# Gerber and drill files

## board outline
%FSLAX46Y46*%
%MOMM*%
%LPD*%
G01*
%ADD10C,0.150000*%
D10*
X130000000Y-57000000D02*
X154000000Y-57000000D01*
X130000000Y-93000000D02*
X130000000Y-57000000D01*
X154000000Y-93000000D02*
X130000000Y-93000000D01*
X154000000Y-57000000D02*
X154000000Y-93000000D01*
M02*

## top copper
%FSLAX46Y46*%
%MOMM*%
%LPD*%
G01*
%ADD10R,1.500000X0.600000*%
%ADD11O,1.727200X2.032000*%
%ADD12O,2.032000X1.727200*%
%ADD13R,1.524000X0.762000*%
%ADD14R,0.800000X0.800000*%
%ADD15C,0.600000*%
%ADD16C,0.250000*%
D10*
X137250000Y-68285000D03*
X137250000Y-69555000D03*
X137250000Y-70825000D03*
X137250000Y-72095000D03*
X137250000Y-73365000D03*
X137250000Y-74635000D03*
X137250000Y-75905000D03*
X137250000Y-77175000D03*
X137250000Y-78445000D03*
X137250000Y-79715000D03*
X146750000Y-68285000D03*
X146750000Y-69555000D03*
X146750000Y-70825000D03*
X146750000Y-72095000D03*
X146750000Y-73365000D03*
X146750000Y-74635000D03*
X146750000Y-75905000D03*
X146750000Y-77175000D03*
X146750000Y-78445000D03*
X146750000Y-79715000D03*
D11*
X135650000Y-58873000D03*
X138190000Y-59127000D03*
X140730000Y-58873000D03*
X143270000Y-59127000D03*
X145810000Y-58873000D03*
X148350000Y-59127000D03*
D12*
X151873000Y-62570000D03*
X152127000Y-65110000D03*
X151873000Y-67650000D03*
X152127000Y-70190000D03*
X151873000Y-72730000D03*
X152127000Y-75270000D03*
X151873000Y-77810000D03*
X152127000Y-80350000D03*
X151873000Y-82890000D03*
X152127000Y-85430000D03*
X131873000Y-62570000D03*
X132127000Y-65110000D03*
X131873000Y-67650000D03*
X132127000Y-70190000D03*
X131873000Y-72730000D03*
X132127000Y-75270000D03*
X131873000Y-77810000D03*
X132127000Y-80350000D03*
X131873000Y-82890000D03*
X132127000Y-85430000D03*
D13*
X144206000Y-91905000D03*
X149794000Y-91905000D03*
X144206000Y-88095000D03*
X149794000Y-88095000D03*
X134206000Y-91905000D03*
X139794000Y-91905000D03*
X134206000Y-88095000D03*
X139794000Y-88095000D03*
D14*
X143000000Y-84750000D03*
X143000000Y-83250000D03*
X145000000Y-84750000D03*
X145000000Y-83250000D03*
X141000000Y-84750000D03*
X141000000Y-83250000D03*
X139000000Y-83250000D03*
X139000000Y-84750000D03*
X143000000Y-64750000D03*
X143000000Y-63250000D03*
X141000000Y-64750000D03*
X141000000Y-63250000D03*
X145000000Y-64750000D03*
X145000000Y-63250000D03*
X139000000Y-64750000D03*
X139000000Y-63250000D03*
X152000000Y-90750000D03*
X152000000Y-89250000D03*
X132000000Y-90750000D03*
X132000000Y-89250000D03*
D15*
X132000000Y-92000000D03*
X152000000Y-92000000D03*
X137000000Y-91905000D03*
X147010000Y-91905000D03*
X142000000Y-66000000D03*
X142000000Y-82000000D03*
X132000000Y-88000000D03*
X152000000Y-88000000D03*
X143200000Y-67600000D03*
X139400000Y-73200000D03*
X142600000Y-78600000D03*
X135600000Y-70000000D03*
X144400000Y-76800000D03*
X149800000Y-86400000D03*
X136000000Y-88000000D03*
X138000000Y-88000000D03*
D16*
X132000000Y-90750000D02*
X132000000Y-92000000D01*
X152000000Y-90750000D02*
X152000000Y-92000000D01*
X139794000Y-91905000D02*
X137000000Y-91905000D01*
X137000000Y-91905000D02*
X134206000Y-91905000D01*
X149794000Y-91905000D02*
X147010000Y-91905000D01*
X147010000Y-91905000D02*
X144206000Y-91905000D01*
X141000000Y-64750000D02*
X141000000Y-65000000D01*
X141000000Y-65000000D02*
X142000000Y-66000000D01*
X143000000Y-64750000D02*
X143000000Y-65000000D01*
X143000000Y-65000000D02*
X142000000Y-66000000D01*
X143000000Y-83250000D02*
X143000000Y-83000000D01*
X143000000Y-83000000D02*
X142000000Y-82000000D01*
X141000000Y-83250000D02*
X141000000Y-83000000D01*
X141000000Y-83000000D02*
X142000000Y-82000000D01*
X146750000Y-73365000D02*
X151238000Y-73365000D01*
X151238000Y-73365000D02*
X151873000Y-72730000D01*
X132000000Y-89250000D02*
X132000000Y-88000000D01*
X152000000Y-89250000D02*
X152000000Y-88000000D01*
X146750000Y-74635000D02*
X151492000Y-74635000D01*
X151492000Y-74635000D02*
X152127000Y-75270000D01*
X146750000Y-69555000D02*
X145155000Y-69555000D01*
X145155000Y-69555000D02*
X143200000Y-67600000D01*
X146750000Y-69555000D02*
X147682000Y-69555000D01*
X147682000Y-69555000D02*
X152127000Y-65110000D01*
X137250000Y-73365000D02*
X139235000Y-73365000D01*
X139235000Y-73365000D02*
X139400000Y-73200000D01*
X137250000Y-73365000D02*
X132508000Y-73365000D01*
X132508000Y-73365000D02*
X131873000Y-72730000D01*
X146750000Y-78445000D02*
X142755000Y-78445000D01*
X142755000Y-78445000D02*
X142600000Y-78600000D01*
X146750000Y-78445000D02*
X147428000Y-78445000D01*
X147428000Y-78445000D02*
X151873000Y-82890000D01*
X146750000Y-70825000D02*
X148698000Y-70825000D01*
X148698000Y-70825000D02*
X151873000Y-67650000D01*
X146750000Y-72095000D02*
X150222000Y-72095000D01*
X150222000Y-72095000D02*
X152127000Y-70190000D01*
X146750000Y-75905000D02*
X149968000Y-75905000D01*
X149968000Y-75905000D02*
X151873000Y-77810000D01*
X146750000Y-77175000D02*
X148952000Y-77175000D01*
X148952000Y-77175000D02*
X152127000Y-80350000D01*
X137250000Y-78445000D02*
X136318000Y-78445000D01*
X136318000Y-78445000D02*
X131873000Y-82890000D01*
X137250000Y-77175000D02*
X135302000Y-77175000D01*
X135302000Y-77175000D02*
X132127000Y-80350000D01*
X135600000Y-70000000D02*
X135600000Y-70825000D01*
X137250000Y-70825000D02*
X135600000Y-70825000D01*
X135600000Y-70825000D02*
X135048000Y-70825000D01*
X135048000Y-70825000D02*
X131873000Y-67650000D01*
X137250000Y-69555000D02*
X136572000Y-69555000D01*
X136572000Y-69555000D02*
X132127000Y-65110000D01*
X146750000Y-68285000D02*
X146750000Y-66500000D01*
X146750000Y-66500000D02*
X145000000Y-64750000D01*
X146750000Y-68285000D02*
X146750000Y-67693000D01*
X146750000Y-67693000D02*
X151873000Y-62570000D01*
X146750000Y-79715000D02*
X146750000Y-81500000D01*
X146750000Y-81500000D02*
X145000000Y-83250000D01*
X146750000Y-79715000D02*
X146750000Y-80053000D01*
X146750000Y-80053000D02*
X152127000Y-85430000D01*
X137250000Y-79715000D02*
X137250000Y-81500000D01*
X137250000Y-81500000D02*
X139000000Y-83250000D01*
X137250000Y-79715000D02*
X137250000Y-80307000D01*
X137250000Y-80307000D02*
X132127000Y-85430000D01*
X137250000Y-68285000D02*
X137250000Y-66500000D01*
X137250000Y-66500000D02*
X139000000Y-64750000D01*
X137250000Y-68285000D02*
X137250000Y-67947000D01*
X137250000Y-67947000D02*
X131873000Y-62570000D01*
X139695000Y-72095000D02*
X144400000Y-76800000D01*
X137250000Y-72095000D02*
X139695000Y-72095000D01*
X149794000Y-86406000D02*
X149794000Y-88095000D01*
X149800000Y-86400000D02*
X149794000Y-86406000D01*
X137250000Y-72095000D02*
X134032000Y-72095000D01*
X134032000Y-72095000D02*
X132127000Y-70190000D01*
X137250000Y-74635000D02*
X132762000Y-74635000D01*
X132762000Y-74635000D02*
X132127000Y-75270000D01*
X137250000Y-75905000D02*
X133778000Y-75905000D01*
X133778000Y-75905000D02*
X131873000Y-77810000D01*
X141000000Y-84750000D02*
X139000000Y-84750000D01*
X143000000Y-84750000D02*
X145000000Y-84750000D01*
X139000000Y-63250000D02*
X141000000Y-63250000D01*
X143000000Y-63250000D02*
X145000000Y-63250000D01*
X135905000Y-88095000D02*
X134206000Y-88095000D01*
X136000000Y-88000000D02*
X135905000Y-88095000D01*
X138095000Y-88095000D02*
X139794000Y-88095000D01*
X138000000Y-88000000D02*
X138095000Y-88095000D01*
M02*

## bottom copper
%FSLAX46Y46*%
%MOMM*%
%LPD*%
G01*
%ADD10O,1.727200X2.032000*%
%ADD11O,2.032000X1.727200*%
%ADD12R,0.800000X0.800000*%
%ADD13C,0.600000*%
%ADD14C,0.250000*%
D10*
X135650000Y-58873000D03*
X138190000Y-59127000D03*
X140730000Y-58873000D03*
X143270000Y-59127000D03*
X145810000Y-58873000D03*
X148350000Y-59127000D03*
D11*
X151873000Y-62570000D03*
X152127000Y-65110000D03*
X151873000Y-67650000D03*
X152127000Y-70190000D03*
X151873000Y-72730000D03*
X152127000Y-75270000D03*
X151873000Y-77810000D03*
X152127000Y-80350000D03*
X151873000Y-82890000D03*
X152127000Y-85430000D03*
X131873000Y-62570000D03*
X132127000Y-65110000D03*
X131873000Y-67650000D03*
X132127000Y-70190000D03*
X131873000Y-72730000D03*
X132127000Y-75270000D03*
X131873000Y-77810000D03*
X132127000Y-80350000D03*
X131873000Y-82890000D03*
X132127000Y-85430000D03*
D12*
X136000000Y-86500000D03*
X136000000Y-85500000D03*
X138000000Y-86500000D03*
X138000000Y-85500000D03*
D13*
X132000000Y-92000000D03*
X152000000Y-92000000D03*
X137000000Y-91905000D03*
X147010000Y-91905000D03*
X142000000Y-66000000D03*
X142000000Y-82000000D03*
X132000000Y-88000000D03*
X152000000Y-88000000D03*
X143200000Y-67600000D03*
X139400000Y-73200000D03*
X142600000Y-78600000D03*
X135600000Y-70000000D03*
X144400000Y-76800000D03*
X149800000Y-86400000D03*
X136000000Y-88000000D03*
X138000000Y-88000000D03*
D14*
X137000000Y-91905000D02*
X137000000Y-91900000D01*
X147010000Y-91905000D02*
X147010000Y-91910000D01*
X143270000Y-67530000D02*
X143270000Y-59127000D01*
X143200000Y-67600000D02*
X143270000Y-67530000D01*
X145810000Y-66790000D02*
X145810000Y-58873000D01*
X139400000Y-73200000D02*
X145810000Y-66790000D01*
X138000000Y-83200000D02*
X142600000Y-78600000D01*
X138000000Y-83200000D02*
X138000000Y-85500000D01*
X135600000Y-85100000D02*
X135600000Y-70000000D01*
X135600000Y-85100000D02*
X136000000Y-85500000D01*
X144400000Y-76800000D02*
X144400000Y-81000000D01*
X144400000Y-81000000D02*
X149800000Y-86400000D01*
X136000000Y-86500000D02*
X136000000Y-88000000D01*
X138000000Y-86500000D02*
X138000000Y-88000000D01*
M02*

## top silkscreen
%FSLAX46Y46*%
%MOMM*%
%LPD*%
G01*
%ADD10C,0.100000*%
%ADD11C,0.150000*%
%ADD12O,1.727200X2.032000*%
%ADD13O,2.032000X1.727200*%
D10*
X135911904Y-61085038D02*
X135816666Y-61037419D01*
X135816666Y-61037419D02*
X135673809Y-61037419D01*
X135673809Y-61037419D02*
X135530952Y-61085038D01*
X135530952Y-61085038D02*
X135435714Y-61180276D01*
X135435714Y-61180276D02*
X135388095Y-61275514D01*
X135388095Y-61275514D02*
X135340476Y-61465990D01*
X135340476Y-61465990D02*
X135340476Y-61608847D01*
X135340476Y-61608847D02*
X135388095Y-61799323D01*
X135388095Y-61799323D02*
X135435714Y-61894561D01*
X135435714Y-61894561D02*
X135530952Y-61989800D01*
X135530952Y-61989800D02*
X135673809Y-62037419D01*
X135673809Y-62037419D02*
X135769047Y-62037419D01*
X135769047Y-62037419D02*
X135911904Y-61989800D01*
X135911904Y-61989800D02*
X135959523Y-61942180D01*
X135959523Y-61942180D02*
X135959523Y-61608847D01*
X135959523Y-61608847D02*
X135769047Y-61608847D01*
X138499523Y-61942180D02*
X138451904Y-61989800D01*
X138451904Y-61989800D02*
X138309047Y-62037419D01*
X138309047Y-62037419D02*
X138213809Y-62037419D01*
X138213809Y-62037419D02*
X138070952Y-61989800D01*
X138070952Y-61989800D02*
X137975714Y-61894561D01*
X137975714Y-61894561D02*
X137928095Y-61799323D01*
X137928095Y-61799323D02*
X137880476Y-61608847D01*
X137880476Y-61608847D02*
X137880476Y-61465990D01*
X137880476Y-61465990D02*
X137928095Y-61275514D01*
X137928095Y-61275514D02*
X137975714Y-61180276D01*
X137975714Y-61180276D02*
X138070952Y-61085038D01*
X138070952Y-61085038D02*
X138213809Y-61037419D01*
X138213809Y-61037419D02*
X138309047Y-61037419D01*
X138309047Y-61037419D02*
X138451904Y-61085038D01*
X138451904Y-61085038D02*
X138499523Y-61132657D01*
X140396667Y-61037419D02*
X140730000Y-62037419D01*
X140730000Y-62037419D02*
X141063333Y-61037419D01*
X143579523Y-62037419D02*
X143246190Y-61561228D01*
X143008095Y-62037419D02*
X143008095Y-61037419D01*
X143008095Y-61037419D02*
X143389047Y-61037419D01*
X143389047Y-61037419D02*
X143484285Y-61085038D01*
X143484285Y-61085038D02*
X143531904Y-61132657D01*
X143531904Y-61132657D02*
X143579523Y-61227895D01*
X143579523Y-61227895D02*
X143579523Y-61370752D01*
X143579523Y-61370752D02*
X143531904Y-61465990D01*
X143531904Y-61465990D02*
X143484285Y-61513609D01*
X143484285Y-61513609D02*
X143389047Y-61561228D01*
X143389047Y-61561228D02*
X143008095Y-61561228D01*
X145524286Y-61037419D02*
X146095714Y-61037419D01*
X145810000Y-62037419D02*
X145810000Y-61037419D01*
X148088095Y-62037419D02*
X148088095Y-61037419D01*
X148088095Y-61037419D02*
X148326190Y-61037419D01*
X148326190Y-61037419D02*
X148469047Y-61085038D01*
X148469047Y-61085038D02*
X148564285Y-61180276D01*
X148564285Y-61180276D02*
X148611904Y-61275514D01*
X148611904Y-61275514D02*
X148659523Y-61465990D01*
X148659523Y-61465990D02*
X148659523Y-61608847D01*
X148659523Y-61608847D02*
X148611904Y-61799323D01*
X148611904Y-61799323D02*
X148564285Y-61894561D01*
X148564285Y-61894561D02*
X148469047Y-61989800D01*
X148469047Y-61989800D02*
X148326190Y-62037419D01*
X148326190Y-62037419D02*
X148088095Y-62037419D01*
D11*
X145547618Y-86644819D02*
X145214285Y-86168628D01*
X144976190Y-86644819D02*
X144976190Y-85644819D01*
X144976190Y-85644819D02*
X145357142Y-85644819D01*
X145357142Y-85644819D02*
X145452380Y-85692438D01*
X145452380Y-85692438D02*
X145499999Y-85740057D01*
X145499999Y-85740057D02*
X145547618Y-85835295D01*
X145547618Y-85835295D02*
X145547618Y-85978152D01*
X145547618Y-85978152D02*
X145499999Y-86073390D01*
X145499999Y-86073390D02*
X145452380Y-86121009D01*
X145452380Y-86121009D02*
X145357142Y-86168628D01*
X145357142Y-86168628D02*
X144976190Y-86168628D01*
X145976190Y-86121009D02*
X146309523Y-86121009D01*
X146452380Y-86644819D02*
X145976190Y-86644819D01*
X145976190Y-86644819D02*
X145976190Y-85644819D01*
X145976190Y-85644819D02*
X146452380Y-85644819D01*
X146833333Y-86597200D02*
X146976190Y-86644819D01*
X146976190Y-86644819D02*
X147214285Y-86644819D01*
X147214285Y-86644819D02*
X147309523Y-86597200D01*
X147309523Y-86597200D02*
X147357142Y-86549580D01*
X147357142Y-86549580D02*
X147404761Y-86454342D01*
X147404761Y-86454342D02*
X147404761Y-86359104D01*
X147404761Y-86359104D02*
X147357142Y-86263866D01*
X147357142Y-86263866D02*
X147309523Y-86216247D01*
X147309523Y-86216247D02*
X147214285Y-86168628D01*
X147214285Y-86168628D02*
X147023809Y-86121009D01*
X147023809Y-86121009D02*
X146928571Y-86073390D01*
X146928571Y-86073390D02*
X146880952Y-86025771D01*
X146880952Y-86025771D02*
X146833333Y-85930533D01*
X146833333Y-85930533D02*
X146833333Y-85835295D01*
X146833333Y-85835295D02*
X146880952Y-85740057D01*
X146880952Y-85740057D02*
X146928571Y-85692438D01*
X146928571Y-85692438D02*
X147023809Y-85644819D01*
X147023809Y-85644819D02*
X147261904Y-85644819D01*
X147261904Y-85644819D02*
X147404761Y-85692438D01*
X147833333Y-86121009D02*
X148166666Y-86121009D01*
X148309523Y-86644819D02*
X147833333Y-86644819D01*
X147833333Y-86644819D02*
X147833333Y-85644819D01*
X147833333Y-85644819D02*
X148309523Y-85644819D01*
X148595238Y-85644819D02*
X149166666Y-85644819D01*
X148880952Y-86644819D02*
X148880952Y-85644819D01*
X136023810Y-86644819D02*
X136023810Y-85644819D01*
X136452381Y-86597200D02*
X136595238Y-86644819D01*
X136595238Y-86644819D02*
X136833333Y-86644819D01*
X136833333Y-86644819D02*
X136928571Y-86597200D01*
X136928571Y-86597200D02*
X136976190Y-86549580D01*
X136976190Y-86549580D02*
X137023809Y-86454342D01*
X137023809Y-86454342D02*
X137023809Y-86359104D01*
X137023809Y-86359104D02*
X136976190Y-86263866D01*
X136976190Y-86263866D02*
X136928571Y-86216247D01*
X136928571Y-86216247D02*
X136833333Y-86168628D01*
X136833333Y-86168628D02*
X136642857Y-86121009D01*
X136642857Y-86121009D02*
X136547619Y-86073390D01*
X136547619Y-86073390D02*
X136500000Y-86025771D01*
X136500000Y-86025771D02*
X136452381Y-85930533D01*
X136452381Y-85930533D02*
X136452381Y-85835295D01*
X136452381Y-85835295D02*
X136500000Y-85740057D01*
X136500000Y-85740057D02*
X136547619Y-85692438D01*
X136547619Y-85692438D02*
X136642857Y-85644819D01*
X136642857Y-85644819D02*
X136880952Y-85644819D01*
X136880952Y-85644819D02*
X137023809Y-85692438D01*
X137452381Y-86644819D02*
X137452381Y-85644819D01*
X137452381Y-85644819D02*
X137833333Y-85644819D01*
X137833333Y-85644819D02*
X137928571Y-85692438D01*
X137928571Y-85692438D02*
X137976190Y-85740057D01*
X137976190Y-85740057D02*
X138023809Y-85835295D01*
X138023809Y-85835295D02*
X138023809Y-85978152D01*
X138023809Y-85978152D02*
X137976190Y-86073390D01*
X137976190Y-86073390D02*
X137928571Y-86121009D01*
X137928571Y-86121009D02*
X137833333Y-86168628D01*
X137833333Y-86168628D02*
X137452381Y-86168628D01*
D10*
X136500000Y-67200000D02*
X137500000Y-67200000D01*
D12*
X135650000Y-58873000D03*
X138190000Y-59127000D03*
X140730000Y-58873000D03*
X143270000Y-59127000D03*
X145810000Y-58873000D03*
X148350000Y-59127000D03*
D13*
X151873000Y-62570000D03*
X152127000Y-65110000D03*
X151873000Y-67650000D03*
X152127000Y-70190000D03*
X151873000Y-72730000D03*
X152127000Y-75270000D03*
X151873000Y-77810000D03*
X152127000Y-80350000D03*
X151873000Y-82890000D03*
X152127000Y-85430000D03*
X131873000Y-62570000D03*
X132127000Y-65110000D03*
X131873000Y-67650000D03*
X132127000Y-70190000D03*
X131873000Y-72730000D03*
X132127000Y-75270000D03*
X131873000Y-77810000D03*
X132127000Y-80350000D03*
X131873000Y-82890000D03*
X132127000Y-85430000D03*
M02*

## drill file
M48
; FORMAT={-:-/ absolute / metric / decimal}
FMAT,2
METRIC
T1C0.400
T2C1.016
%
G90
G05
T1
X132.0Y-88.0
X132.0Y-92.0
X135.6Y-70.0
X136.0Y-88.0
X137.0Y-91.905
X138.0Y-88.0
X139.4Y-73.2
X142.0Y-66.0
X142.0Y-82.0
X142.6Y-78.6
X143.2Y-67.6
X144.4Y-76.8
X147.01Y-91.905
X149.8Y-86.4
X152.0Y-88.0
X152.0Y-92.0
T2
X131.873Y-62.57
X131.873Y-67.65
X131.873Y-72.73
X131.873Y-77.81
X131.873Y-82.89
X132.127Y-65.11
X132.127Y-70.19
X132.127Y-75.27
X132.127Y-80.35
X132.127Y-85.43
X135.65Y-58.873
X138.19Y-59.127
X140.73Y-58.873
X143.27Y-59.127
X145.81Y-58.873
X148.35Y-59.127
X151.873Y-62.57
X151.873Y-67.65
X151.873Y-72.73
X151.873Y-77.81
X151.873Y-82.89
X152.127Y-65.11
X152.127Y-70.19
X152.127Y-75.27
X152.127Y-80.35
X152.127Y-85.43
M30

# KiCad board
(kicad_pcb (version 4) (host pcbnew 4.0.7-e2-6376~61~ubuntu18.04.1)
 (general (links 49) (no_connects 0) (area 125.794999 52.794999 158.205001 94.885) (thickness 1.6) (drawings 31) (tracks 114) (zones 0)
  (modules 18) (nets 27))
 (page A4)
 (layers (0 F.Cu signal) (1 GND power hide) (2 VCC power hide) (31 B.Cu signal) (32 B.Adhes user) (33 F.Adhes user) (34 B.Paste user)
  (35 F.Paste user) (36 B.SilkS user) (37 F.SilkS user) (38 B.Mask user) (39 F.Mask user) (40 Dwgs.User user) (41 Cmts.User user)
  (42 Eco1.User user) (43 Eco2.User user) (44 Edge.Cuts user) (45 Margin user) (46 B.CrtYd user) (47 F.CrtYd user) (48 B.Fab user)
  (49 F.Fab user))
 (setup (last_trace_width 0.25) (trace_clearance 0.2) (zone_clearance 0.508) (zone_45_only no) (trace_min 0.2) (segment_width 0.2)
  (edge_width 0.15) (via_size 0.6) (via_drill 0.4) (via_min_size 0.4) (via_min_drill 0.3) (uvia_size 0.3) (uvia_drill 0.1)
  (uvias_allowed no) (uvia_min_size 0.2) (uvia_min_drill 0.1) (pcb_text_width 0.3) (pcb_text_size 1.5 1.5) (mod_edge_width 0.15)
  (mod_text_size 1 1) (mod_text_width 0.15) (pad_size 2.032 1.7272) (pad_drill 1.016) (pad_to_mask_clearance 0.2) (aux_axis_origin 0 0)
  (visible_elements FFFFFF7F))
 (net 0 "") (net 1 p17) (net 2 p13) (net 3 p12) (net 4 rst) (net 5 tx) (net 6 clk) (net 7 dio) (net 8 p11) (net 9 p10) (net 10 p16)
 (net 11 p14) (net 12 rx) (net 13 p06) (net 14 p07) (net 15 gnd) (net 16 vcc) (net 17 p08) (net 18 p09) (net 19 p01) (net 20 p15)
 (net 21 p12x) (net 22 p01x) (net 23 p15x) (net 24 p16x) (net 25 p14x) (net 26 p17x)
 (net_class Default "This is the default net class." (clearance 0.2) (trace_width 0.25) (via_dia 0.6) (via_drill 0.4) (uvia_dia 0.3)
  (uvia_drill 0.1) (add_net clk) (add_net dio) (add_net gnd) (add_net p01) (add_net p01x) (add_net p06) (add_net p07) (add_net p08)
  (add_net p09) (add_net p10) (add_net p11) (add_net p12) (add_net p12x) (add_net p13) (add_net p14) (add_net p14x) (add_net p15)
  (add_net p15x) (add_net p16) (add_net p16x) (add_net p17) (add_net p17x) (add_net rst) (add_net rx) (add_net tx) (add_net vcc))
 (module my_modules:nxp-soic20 (layer F.Cu) (at 142 74)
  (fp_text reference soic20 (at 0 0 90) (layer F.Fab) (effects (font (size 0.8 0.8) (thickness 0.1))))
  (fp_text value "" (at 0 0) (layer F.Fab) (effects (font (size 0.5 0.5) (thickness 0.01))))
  (fp_line (start -5.5 -6.8) (end -4.5 -6.8) (layer F.SilkS) (width 0.1))
  (pad P17 smd rect (at -4.75 -5.715) (size 1.5 0.6) (layers F.Cu F.Paste F.Mask) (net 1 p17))
  (pad P13 smd rect (at -4.75 -4.445) (size 1.5 0.6) (layers F.Cu F.Paste F.Mask) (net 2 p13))
  (pad P12 smd rect (at -4.75 -3.175) (size 1.5 0.6) (layers F.Cu F.Paste F.Mask) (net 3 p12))
  (pad RST smd rect (at -4.75 -1.905) (size 1.5 0.6) (layers F.Cu F.Paste F.Mask) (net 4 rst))
  (pad P04 smd rect (at -4.75 -0.635) (size 1.5 0.6) (layers F.Cu F.Paste F.Mask) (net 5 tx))
  (pad CLK smd rect (at -4.75 0.635) (size 1.5 0.6) (layers F.Cu F.Paste F.Mask) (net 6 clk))
  (pad DIO smd rect (at -4.75 1.905) (size 1.5 0.6) (layers F.Cu F.Paste F.Mask) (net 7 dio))
  (pad P11 smd rect (at -4.75 3.175) (size 1.5 0.6) (layers F.Cu F.Paste F.Mask) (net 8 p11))
  (pad P10 smd rect (at -4.75 4.445) (size 1.5 0.6) (layers F.Cu F.Paste F.Mask) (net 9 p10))
  (pad P16 smd rect (at -4.75 5.715) (size 1.5 0.6) (layers F.Cu F.Paste F.Mask) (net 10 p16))
  (pad P14 smd rect (at 4.75 -5.715) (size 1.5 0.6) (layers F.Cu F.Paste F.Mask) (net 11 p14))
  (pad P00 smd rect (at 4.75 -4.445) (size 1.5 0.6) (layers F.Cu F.Paste F.Mask) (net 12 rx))
  (pad P06 smd rect (at 4.75 -3.175) (size 1.5 0.6) (layers F.Cu F.Paste F.Mask) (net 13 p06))
  (pad P07 smd rect (at 4.75 -1.905) (size 1.5 0.6) (layers F.Cu F.Paste F.Mask) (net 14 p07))
  (pad GND smd rect (at 4.75 -0.635) (size 1.5 0.6) (layers F.Cu F.Paste F.Mask) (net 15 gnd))
  (pad VCC smd rect (at 4.75 0.635) (size 1.5 0.6) (layers F.Cu F.Paste F.Mask) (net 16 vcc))
  (pad P08 smd rect (at 4.75 1.905) (size 1.5 0.6) (layers F.Cu F.Paste F.Mask) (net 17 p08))
  (pad P09 smd rect (at 4.75 3.175) (size 1.5 0.6) (layers F.Cu F.Paste F.Mask) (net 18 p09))
  (pad P01 smd rect (at 4.75 4.445) (size 1.5 0.6) (layers F.Cu F.Paste F.Mask) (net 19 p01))
  (pad P15 smd rect (at 4.75 5.715) (size 1.5 0.6) (layers F.Cu F.Paste F.Mask) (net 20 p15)))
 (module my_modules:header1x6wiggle (layer F.Cu) (at 142 59 90)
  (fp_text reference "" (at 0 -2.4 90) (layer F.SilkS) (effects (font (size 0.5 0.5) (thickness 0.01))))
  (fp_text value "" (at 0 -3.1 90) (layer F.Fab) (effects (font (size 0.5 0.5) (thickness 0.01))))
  (pad GND thru_hole oval (at 0.127 -6.35 90) (size 2.032 1.7272) (drill 1.016) (layers *.Cu *.Mask F.SilkS) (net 15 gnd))
  (pad CTS thru_hole oval (at -0.127 -3.81 90) (size 2.032 1.7272) (drill 1.016) (layers *.Cu *.Mask F.SilkS))
  (pad VCC thru_hole oval (at 0.127 -1.27 90) (size 2.032 1.7272) (drill 1.016) (layers *.Cu *.Mask F.SilkS) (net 16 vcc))
  (pad TX thru_hole oval (at -0.127 1.27 90) (size 2.032 1.7272) (drill 1.016) (layers *.Cu *.Mask F.SilkS) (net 12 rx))
  (pad RX thru_hole oval (at 0.127 3.81 90) (size 2.032 1.7272) (drill 1.016) (layers *.Cu *.Mask F.SilkS) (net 5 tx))
  (pad DTR thru_hole oval (at -0.127 6.35 90) (size 2.032 1.7272) (drill 1.016) (layers *.Cu *.Mask F.SilkS)))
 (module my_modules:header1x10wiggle (layer F.Cu) (at 152 74)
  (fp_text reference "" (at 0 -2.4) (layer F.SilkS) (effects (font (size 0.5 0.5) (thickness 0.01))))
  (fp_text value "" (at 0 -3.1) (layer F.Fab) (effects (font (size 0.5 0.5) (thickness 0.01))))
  (pad P14 thru_hole oval (at -0.127 -11.43) (size 2.032 1.7272) (drill 1.016) (layers *.Cu *.Mask F.SilkS) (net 11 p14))
  (pad P00 thru_hole oval (at 0.127 -8.89) (size 2.032 1.7272) (drill 1.016) (layers *.Cu *.Mask F.SilkS) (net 12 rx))
  (pad P06 thru_hole oval (at -0.127 -6.35) (size 2.032 1.7272) (drill 1.016) (layers *.Cu *.Mask F.SilkS) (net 13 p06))
  (pad P07 thru_hole oval (at 0.127 -3.81) (size 2.032 1.7272) (drill 1.016) (layers *.Cu *.Mask F.SilkS) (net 14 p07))
  (pad GND thru_hole oval (at -0.127 -1.27) (size 2.032 1.7272) (drill 1.016) (layers *.Cu *.Mask F.SilkS) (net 15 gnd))
  (pad VCC thru_hole oval (at 0.127 1.27) (size 2.032 1.7272) (drill 1.016) (layers *.Cu *.Mask F.SilkS) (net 16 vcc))
  (pad P08 thru_hole oval (at -0.127 3.81) (size 2.032 1.7272) (drill 1.016) (layers *.Cu *.Mask F.SilkS) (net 17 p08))
  (pad P09 thru_hole oval (at 0.127 6.35) (size 2.032 1.7272) (drill 1.016) (layers *.Cu *.Mask F.SilkS) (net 18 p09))
  (pad P01 thru_hole oval (at -0.127 8.89) (size 2.032 1.7272) (drill 1.016) (layers *.Cu *.Mask F.SilkS) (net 19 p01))
  (pad P15 thru_hole oval (at 0.127 11.43) (size 2.032 1.7272) (drill 1.016) (layers *.Cu *.Mask F.SilkS) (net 20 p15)))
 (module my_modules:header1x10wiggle (layer F.Cu) (at 132 74)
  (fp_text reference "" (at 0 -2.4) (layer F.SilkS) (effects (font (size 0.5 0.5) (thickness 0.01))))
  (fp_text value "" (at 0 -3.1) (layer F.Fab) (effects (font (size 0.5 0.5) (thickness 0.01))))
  (pad P17 thru_hole oval (at -0.127 -11.43) (size 2.032 1.7272) (drill 1.016) (layers *.Cu *.Mask F.SilkS) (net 1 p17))
  (pad P13 thru_hole oval (at 0.127 -8.89) (size 2.032 1.7272) (drill 1.016) (layers *.Cu *.Mask F.SilkS) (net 2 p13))
  (pad P12 thru_hole oval (at -0.127 -6.35) (size 2.032 1.7272) (drill 1.016) (layers *.Cu *.Mask F.SilkS) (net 3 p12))
  (pad RST thru_hole oval (at 0.127 -3.81) (size 2.032 1.7272) (drill 1.016) (layers *.Cu *.Mask F.SilkS) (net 4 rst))
  (pad P04 thru_hole oval (at -0.127 -1.27) (size 2.032 1.7272) (drill 1.016) (layers *.Cu *.Mask F.SilkS) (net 5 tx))
  (pad CLK thru_hole oval (at 0.127 1.27) (size 2.032 1.7272) (drill 1.016) (layers *.Cu *.Mask F.SilkS) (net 6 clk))
  (pad DIO thru_hole oval (at -0.127 3.81) (size 2.032 1.7272) (drill 1.016) (layers *.Cu *.Mask F.SilkS) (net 7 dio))
  (pad P11 thru_hole oval (at 0.127 6.35) (size 2.032 1.7272) (drill 1.016) (layers *.Cu *.Mask F.SilkS) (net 8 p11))
  (pad P10 thru_hole oval (at -0.127 8.89) (size 2.032 1.7272) (drill 1.016) (layers *.Cu *.Mask F.SilkS) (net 9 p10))
  (pad P16 thru_hole oval (at 0.127 11.43) (size 2.032 1.7272) (drill 1.016) (layers *.Cu *.Mask F.SilkS) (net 10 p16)))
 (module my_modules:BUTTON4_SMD (layer F.Cu) (at 147 90)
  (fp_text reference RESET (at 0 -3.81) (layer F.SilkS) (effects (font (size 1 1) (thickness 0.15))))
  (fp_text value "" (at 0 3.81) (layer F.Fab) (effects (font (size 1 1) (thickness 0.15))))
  (pad 1 smd rect (at -2.794 1.905) (size 1.524 0.762) (layers F.Cu F.Paste F.Mask) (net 15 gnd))
  (pad 2 smd rect (at 2.794 1.905) (size 1.524 0.762) (layers F.Cu F.Paste F.Mask) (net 15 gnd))
  (pad 3 smd rect (at -2.794 -1.905) (size 1.524 0.762) (layers F.Cu F.Paste F.Mask))
  (pad 4 smd rect (at 2.794 -1.905) (size 1.524 0.762) (layers F.Cu F.Paste F.Mask) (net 4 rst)))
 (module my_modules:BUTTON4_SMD (layer F.Cu) (at 137 90)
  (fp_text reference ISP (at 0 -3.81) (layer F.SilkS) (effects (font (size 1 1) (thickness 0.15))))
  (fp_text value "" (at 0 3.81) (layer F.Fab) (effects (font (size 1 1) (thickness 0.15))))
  (pad 1 smd rect (at -2.794 1.905) (size 1.524 0.762) (layers F.Cu F.Paste F.Mask) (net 15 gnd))
  (pad 2 smd rect (at 2.794 1.905) (size 1.524 0.762) (layers F.Cu F.Paste F.Mask) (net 15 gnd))
  (pad 3 smd rect (at -2.794 -1.905) (size 1.524 0.762) (layers F.Cu F.Paste F.Mask) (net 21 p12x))
  (pad 4 smd rect (at 2.794 -1.905) (size 1.524 0.762) (layers F.Cu F.Paste F.Mask) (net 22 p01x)))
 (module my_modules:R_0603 (layer F.Cu) (at 143 84 90)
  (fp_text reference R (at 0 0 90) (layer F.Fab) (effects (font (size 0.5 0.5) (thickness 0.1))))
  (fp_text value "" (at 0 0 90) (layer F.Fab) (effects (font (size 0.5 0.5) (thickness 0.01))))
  (pad 1 smd rect (at -0.75 0 90) (size 0.8 0.8) (layers F.Cu F.Paste F.Mask) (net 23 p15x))
  (pad 2 smd rect (at 0.75 0 90) (size 0.8 0.8) (layers F.Cu F.Paste F.Mask) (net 15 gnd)))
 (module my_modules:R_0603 (layer F.Cu) (at 145 84 90)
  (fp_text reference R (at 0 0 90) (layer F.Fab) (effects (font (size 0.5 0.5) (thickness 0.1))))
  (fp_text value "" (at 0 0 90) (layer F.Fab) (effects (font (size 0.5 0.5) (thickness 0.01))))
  (pad 1 smd rect (at -0.75 0 90) (size 0.8 0.8) (layers F.Cu F.Paste F.Mask) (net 23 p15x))
  (pad 2 smd rect (at 0.75 0 90) (size 0.8 0.8) (layers F.Cu F.Paste F.Mask) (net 20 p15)))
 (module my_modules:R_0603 (layer F.Cu) (at 141 84 90)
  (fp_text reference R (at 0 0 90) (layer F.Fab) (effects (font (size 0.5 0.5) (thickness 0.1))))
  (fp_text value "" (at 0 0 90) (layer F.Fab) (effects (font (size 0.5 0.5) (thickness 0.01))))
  (pad 1 smd rect (at -0.75 0 90) (size 0.8 0.8) (layers F.Cu F.Paste F.Mask) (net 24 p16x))
  (pad 2 smd rect (at 0.75 0 90) (size 0.8 0.8) (layers F.Cu F.Paste F.Mask) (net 15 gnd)))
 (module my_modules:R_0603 (layer F.Cu) (at 139 84 270)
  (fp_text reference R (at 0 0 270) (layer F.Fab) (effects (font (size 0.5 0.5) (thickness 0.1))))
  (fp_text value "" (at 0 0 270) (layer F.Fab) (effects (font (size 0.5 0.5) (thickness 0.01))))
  (pad 1 smd rect (at -0.75 0 270) (size 0.8 0.8) (layers F.Cu F.Paste F.Mask) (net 10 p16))
  (pad 2 smd rect (at 0.75 0 270) (size 0.8 0.8) (layers F.Cu F.Paste F.Mask) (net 24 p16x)))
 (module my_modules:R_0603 (layer F.Cu) (at 143 64 90)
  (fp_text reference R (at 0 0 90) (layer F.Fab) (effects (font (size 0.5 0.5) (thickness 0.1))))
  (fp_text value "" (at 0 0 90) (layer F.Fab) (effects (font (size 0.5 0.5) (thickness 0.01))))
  (pad 1 smd rect (at -0.75 0 90) (size 0.8 0.8) (layers F.Cu F.Paste F.Mask) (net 15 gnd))
  (pad 2 smd rect (at 0.75 0 90) (size 0.8 0.8) (layers F.Cu F.Paste F.Mask) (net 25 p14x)))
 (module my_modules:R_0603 (layer F.Cu) (at 141 64 90)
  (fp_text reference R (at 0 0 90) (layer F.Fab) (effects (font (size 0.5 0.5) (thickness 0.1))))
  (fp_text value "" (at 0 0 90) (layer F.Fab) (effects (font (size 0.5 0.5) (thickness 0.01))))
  (pad 1 smd rect (at -0.75 0 90) (size 0.8 0.8) (layers F.Cu F.Paste F.Mask) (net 15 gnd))
  (pad 2 smd rect (at 0.75 0 90) (size 0.8 0.8) (layers F.Cu F.Paste F.Mask) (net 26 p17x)))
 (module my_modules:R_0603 (layer F.Cu) (at 145 64 90)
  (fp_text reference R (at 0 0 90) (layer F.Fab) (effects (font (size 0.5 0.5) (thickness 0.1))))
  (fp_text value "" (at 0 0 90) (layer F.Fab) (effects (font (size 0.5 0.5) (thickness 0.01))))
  (pad 1 smd rect (at -0.75 0 90) (size 0.8 0.8) (layers F.Cu F.Paste F.Mask) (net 11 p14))
  (pad 2 smd rect (at 0.75 0 90) (size 0.8 0.8) (layers F.Cu F.Paste F.Mask) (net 25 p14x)))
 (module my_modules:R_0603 (layer F.Cu) (at 139 64 90)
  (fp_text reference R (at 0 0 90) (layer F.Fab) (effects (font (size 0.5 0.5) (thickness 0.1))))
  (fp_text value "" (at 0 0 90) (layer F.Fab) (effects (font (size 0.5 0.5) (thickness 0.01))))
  (pad 1 smd rect (at -0.75 0 90) (size 0.8 0.8) (layers F.Cu F.Paste F.Mask) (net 1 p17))
  (pad 2 smd rect (at 0.75 0 90) (size 0.8 0.8) (layers F.Cu F.Paste F.Mask) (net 26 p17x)))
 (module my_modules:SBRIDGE (layer B.Cu) (at 136 86 90)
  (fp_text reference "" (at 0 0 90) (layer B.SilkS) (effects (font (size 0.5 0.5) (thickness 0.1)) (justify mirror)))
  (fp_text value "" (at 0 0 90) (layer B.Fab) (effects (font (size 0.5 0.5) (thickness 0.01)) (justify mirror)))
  (pad 1 smd rect (at -0.5 0 90) (size 0.8 0.8) (layers B.Cu B.Paste B.Mask) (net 21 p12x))
  (pad 2 smd rect (at 0.5 0 90) (size 0.8 0.8) (layers B.Cu B.Paste B.Mask) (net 3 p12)))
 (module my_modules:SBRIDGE (layer B.Cu) (at 138 86 90)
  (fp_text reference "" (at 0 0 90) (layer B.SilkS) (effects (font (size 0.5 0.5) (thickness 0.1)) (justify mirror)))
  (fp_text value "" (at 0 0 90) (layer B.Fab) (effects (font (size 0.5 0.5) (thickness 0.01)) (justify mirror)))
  (pad 1 smd rect (at -0.5 0 90) (size 0.8 0.8) (layers B.Cu B.Paste B.Mask) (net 22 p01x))
  (pad 2 smd rect (at 0.5 0 90) (size 0.8 0.8) (layers B.Cu B.Paste B.Mask) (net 19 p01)))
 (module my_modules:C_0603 (layer F.Cu) (at 152 90 90)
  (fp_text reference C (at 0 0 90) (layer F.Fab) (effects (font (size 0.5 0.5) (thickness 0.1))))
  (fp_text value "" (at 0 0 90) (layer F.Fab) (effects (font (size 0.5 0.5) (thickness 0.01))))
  (pad 1 smd rect (at -0.75 0 90) (size 0.8 0.8) (layers F.Cu F.Paste F.Mask) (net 15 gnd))
  (pad 2 smd rect (at 0.75 0 90) (size 0.8 0.8) (layers F.Cu F.Paste F.Mask) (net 16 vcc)))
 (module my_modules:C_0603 (layer F.Cu) (at 132 90 90)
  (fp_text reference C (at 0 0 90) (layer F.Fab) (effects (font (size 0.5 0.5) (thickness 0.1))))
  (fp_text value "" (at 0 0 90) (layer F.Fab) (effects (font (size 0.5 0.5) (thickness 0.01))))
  (pad 1 smd rect (at -0.75 0 90) (size 0.8 0.8) (layers F.Cu F.Paste F.Mask) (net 15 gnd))
  (pad 2 smd rect (at 0.75 0 90) (size 0.8 0.8) (layers F.Cu F.Paste F.Mask) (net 16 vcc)))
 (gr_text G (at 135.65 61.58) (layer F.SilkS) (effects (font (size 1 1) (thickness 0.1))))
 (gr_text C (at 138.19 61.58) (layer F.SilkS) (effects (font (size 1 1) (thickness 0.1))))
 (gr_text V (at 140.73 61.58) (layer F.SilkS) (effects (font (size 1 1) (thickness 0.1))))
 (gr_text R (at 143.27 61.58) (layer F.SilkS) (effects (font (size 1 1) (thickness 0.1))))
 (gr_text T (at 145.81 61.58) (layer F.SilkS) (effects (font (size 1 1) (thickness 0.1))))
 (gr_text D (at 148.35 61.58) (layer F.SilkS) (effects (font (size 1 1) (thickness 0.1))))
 (gr_line (start 130 57) (end 154 57) (angle 90) (layer Edge.Cuts) (width 0.15))
 (gr_line (start 130 93) (end 130 57) (angle 90) (layer Edge.Cuts) (width 0.15))
 (gr_line (start 154 93) (end 130 93) (angle 90) (layer Edge.Cuts) (width 0.15))
 (gr_line (start 154 57) (end 154 93) (angle 90) (layer Edge.Cuts) (width 0.15))
 (segment (start 132 90.75) (end 132 92) (width 0.25) (layer F.Cu) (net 15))
 (via (at 132 92) (size 0.6) (drill 0.4) (layers F.Cu B.Cu) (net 15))
 (segment (start 152 90.75) (end 152 92) (width 0.25) (layer F.Cu) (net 15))
 (via (at 152 92) (size 0.6) (drill 0.4) (layers F.Cu B.Cu) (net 15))
 (via (at 137 91.905) (size 0.6) (drill 0.4) (layers F.Cu B.Cu) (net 15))
 (segment (start 137 91.905) (end 137 91.9) (width 0.25) (layer B.Cu) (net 15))
 (segment (start 139.794 91.905) (end 137 91.905) (width 0.25) (layer F.Cu) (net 15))
 (segment (start 137 91.905) (end 134.206 91.905) (width 0.25) (layer F.Cu) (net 15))
 (via (at 147.01 91.905) (size 0.6) (drill 0.4) (layers F.Cu B.Cu) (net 15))
 (segment (start 147.01 91.905) (end 147.01 91.91) (width 0.25) (layer B.Cu) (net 15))
 (segment (start 149.794 91.905) (end 147.01 91.905) (width 0.25) (layer F.Cu) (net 15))
 (segment (start 147.01 91.905) (end 144.206 91.905) (width 0.25) (layer F.Cu) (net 15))
 (segment (start 141 64.75) (end 141 65) (width 0.25) (layer F.Cu) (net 15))
 (segment (start 141 65) (end 142 66) (width 0.25) (layer F.Cu) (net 15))
 (segment (start 143 64.75) (end 143 65) (width 0.25) (layer F.Cu) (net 15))
 (segment (start 143 65) (end 142 66) (width 0.25) (layer F.Cu) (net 15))
 (via (at 142 66) (size 0.6) (drill 0.4) (layers F.Cu B.Cu) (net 15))
 (segment (start 143 83.25) (end 143 83) (width 0.25) (layer F.Cu) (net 15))
 (segment (start 143 83) (end 142 82) (width 0.25) (layer F.Cu) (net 15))
 (segment (start 141 83.25) (end 141 83) (width 0.25) (layer F.Cu) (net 15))
 (segment (start 141 83) (end 142 82) (width 0.25) (layer F.Cu) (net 15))
 (via (at 142 82) (size 0.6) (drill 0.4) (layers F.Cu B.Cu) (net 15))
 (segment (start 146.75 73.365) (end 151.238 73.365) (width 0.25) (layer F.Cu) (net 15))
 (segment (start 151.238 73.365) (end 151.873 72.73) (width 0.25) (layer F.Cu) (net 15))
 (segment (start 132 89.25) (end 132 88) (width 0.25) (layer F.Cu) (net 16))
 (via (at 132 88) (size 0.6) (drill 0.4) (layers F.Cu B.Cu) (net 16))
 (via (at 152 88) (size 0.6) (drill 0.4) (layers F.Cu B.Cu) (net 16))
 (segment (start 152 89.25) (end 152 88) (width 0.25) (layer F.Cu) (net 16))
 (segment (start 146.75 74.635) (end 151.492 74.635) (width 0.25) (layer F.Cu) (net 16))
 (segment (start 151.492 74.635) (end 152.127 75.27) (width 0.25) (layer F.Cu) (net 16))
 (segment (start 146.75 69.555) (end 145.155 69.555) (width 0.25) (layer F.Cu) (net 12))
 (segment (start 143.27 67.53) (end 143.27 59.127) (width 0.25) (layer B.Cu) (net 12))
 (segment (start 143.2 67.6) (end 143.27 67.53) (width 0.25) (layer B.Cu) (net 12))
 (via (at 143.2 67.6) (size 0.6) (drill 0.4) (layers F.Cu B.Cu) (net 12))
 (segment (start 145.155 69.555) (end 143.2 67.6) (width 0.25) (layer F.Cu) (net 12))
 (segment (start 146.75 69.555) (end 147.682 69.555) (width 0.25) (layer F.Cu) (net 12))
 (segment (start 147.682 69.555) (end 152.127 65.11) (width 0.25) (layer F.Cu) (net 12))
 (segment (start 137.25 73.365) (end 139.235 73.365) (width 0.25) (layer F.Cu) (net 5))
 (segment (start 145.81 66.79) (end 145.81 58.873) (width 0.25) (layer B.Cu) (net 5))
 (segment (start 139.4 73.2) (end 145.81 66.79) (width 0.25) (layer B.Cu) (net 5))
 (via (at 139.4 73.2) (size 0.6) (drill 0.4) (layers F.Cu B.Cu) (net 5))
 (segment (start 139.235 73.365) (end 139.4 73.2) (width 0.25) (layer F.Cu) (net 5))
 (segment (start 137.25 73.365) (end 132.508 73.365) (width 0.25) (layer F.Cu) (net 5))
 (segment (start 132.508 73.365) (end 131.873 72.73) (width 0.25) (layer F.Cu) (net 5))
 (segment (start 146.75 78.445) (end 142.755 78.445) (width 0.25) (layer F.Cu) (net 19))
 (segment (start 138 83.2) (end 142.6 78.6) (width 0.25) (layer B.Cu) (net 19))
 (via (at 142.6 78.6) (size 0.6) (drill 0.4) (layers F.Cu B.Cu) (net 19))
 (segment (start 138 83.2) (end 138 85.5) (width 0.25) (layer B.Cu) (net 19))
 (segment (start 142.755 78.445) (end 142.6 78.6) (width 0.25) (layer F.Cu) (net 19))
 (segment (start 146.75 78.445) (end 147.428 78.445) (width 0.25) (layer F.Cu) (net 19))
 (segment (start 147.428 78.445) (end 151.873 82.89) (width 0.25) (layer F.Cu) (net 19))
 (segment (start 146.75 70.825) (end 148.698 70.825) (width 0.25) (layer F.Cu) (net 13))
 (segment (start 148.698 70.825) (end 151.873 67.65) (width 0.25) (layer F.Cu) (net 13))
 (segment (start 146.75 72.095) (end 150.222 72.095) (width 0.25) (layer F.Cu) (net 14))
 (segment (start 150.222 72.095) (end 152.127 70.19) (width 0.25) (layer F.Cu) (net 14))
 (segment (start 146.75 75.905) (end 149.968 75.905) (width 0.25) (layer F.Cu) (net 17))
 (segment (start 149.968 75.905) (end 151.873 77.81) (width 0.25) (layer F.Cu) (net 17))
 (segment (start 146.75 77.175) (end 148.952 77.175) (width 0.25) (layer F.Cu) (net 18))
 (segment (start 148.952 77.175) (end 152.127 80.35) (width 0.25) (layer F.Cu) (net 18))
 (segment (start 137.25 78.445) (end 136.318 78.445) (width 0.25) (layer F.Cu) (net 9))
 (segment (start 136.318 78.445) (end 131.873 82.89) (width 0.25) (layer F.Cu) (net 9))
 (segment (start 137.25 77.175) (end 135.302 77.175) (width 0.25) (layer F.Cu) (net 8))
 (segment (start 135.302 77.175) (end 132.127 80.35) (width 0.25) (layer F.Cu) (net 8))
 (segment (start 135.6 85.1) (end 135.6 70) (width 0.25) (layer B.Cu) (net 3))
 (via (at 135.6 70) (size 0.6) (drill 0.4) (layers F.Cu B.Cu) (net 3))
 (segment (start 135.6 70) (end 135.6 70.825) (width 0.25) (layer F.Cu) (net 3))
 (segment (start 135.6 85.1) (end 136 85.5) (width 0.25) (layer B.Cu) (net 3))
 (segment (start 137.25 70.825) (end 135.6 70.825) (width 0.25) (layer F.Cu) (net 3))
 (segment (start 135.6 70.825) (end 135.048 70.825) (width 0.25) (layer F.Cu) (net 3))
 (segment (start 135.048 70.825) (end 131.873 67.65) (width 0.25) (layer F.Cu) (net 3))
 (segment (start 137.25 69.555) (end 136.572 69.555) (width 0.25) (layer F.Cu) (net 2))
 (segment (start 136.572 69.555) (end 132.127 65.11) (width 0.25) (layer F.Cu) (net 2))
 (segment (start 146.75 68.285) (end 146.75 66.5) (width 0.25) (layer F.Cu) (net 11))
 (segment (start 146.75 66.5) (end 145 64.75) (width 0.25) (layer F.Cu) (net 11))
 (segment (start 146.75 68.285) (end 146.75 67.693) (width 0.25) (layer F.Cu) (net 11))
 (segment (start 146.75 67.693) (end 151.873 62.57) (width 0.25) (layer F.Cu) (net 11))
 (segment (start 146.75 79.715) (end 146.75 81.5) (width 0.25) (layer F.Cu) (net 20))
 (segment (start 146.75 81.5) (end 145 83.25) (width 0.25) (layer F.Cu) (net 20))
 (segment (start 146.75 79.715) (end 146.75 80.053) (width 0.25) (layer F.Cu) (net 20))
 (segment (start 146.75 80.053) (end 152.127 85.43) (width 0.25) (layer F.Cu) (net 20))
 (segment (start 137.25 79.715) (end 137.25 81.5) (width 0.25) (layer F.Cu) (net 10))
 (segment (start 137.25 81.5) (end 139 83.25) (width 0.25) (layer F.Cu) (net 10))
 (segment (start 137.25 79.715) (end 137.25 80.307) (width 0.25) (layer F.Cu) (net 10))
 (segment (start 137.25 80.307) (end 132.127 85.43) (width 0.25) (layer F.Cu) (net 10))
 (segment (start 137.25 68.285) (end 137.25 66.5) (width 0.25) (layer F.Cu) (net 1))
 (segment (start 137.25 66.5) (end 139 64.75) (width 0.25) (layer F.Cu) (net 1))
 (segment (start 137.25 68.285) (end 137.25 67.947) (width 0.25) (layer F.Cu) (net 1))
 (segment (start 137.25 67.947) (end 131.873 62.57) (width 0.25) (layer F.Cu) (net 1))
 (segment (start 144.4 76.8) (end 144.4 81) (width 0.25) (layer B.Cu) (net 4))
 (segment (start 139.695 72.095) (end 144.4 76.8) (width 0.25) (layer F.Cu) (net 4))
 (via (at 144.4 76.8) (size 0.6) (drill 0.4) (layers F.Cu B.Cu) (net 4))
 (segment (start 137.25 72.095) (end 139.695 72.095) (width 0.25) (layer F.Cu) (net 4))
 (segment (start 149.794 86.406) (end 149.794 88.095) (width 0.25) (layer F.Cu) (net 4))
 (segment (start 149.8 86.4) (end 149.794 86.406) (width 0.25) (layer F.Cu) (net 4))
 (via (at 149.8 86.4) (size 0.6) (drill 0.4) (layers F.Cu B.Cu) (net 4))
 (segment (start 144.4 81) (end 149.8 86.4) (width 0.25) (layer B.Cu) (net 4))
 (segment (start 137.25 72.095) (end 134.032 72.095) (width 0.25) (layer F.Cu) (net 4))
 (segment (start 134.032 72.095) (end 132.127 70.19) (width 0.25) (layer F.Cu) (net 4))
 (segment (start 137.25 74.635) (end 132.762 74.635) (width 0.25) (layer F.Cu) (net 6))
 (segment (start 132.762 74.635) (end 132.127 75.27) (width 0.25) (layer F.Cu) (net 6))
 (segment (start 137.25 75.905) (end 133.778 75.905) (width 0.25) (layer F.Cu) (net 7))
 (segment (start 133.778 75.905) (end 131.873 77.81) (width 0.25) (layer F.Cu) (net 7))
 (segment (start 141 84.75) (end 139 84.75) (width 0.25) (layer F.Cu) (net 24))
 (segment (start 143 84.75) (end 145 84.75) (width 0.25) (layer F.Cu) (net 23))
 (segment (start 139 63.25) (end 141 63.25) (width 0.25) (layer F.Cu) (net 26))
 (segment (start 143 63.25) (end 145 63.25) (width 0.25) (layer F.Cu) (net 25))
 (segment (start 136 86.5) (end 136 88) (width 0.25) (layer B.Cu) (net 21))
 (segment (start 135.905 88.095) (end 134.206 88.095) (width 0.25) (layer F.Cu) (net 21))
 (segment (start 136 88) (end 135.905 88.095) (width 0.25) (layer F.Cu) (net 21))
 (via (at 136 88) (size 0.6) (drill 0.4) (layers F.Cu B.Cu) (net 21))
 (segment (start 138 86.5) (end 138 88) (width 0.25) (layer B.Cu) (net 22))
 (segment (start 138.095 88.095) (end 139.794 88.095) (width 0.25) (layer F.Cu) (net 22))
 (segment (start 138 88) (end 138.095 88.095) (width 0.25) (layer F.Cu) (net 22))
 (via (at 138 88) (size 0.6) (drill 0.4) (layers F.Cu B.Cu) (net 22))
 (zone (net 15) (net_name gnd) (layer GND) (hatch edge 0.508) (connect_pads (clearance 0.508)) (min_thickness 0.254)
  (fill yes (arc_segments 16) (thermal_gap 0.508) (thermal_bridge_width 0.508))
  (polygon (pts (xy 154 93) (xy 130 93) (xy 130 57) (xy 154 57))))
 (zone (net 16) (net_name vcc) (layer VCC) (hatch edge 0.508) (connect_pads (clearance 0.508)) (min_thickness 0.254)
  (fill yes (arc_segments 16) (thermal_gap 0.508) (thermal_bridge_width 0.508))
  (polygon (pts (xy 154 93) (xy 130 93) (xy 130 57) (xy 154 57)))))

